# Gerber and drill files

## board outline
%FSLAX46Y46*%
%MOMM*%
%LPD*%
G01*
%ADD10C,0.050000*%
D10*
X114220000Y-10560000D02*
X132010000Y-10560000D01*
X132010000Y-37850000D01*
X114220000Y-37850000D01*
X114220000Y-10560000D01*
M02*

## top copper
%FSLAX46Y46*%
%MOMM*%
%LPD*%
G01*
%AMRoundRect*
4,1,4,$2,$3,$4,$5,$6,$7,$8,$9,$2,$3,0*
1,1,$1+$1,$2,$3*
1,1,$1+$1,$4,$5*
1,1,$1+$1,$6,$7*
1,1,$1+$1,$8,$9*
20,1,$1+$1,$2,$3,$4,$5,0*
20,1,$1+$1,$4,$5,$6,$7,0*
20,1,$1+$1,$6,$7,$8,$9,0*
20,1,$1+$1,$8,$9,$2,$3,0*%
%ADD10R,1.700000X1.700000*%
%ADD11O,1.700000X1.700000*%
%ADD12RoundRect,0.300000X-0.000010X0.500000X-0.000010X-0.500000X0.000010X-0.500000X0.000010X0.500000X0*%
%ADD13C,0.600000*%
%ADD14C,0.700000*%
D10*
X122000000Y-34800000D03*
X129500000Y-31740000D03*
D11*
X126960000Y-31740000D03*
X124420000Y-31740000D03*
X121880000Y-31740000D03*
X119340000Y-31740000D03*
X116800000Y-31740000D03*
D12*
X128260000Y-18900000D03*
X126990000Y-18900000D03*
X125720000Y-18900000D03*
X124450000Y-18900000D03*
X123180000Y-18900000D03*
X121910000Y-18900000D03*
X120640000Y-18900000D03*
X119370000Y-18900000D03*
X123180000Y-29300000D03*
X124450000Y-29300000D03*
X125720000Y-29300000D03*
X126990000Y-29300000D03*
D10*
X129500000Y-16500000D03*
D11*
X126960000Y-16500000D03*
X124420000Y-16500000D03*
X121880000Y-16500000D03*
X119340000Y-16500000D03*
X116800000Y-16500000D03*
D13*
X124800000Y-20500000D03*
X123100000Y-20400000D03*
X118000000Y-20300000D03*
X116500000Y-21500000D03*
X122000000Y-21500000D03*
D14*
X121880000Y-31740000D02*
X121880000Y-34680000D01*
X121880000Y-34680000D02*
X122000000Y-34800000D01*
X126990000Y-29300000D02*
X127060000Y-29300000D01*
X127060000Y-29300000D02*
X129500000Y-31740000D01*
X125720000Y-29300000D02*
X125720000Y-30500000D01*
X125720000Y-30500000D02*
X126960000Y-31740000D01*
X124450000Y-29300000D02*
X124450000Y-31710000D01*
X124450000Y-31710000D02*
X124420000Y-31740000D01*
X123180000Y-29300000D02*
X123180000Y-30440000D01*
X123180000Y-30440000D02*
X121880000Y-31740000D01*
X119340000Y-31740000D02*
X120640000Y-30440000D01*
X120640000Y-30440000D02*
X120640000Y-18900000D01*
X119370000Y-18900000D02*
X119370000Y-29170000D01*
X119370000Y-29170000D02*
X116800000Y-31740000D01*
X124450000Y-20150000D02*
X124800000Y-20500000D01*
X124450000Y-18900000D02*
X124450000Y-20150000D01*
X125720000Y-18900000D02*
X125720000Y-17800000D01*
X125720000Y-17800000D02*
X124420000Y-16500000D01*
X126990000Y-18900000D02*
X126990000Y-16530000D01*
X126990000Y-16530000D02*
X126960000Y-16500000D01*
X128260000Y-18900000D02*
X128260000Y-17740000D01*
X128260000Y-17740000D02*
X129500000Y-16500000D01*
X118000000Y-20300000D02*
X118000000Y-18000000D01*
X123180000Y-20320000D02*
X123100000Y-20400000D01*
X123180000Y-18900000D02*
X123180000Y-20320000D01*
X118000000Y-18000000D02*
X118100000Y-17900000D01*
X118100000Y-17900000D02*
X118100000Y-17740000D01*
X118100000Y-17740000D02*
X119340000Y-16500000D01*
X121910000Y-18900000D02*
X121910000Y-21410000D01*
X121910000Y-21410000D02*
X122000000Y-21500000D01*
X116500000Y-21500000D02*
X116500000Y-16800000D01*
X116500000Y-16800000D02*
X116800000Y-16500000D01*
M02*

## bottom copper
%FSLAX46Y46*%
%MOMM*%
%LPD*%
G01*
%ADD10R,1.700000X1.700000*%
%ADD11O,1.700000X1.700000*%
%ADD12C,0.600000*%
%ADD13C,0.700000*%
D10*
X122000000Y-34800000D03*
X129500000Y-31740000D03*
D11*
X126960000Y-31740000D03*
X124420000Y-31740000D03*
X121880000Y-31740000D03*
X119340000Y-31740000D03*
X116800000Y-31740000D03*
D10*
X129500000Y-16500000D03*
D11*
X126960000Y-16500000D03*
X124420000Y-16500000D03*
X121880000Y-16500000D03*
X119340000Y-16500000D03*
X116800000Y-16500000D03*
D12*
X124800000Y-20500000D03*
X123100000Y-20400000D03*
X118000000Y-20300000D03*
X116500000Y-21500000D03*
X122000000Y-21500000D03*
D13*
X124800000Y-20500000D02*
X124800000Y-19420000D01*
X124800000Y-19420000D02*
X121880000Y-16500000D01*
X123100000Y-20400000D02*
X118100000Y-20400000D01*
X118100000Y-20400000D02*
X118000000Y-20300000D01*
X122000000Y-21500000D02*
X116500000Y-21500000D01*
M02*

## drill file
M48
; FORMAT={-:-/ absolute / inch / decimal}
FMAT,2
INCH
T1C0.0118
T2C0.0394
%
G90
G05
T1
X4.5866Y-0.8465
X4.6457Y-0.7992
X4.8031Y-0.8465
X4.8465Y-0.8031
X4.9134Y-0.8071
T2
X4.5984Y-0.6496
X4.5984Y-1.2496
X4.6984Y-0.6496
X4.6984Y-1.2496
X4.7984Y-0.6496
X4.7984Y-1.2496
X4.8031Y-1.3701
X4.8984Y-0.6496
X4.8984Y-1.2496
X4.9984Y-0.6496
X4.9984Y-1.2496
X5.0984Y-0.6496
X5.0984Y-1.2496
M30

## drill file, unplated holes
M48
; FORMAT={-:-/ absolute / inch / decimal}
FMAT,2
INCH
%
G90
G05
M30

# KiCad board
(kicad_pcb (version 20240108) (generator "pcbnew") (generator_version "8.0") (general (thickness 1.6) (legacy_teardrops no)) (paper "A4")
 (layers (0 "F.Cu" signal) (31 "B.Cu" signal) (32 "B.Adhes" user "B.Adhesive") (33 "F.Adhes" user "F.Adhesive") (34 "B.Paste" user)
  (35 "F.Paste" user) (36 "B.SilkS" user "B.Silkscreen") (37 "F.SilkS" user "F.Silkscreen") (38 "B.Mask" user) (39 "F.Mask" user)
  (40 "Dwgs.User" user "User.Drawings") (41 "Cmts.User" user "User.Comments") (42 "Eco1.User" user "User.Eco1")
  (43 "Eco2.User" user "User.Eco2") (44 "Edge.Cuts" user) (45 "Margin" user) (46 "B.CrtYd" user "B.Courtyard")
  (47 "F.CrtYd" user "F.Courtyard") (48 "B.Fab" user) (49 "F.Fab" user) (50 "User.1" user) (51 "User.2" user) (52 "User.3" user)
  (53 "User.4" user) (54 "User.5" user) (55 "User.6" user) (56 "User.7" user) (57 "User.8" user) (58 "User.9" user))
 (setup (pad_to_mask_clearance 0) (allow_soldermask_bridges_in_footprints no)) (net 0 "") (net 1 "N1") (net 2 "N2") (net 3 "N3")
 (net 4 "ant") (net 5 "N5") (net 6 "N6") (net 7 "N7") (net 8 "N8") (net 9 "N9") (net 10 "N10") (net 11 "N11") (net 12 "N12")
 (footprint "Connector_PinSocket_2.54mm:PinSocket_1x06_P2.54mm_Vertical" (layer "F.Cu") (at 129.5 31.74 -90)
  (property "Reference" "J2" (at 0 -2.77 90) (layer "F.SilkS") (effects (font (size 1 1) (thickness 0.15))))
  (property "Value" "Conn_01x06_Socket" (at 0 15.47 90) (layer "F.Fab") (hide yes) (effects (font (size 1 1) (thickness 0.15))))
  (pad "1" thru_hole rect (at 0 0 270) (size 1.7 1.7) (drill 1) (layers "*.Cu" "*.Mask") (remove_unused_layers no) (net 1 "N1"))
  (pad "2" thru_hole oval (at 0 2.54 270) (size 1.7 1.7) (drill 1) (layers "*.Cu" "*.Mask") (remove_unused_layers no) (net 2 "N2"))
  (pad "3" thru_hole oval (at 0 5.08 270) (size 1.7 1.7) (drill 1) (layers "*.Cu" "*.Mask") (remove_unused_layers no) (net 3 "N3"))
  (pad "4" thru_hole oval (at 0 7.62 270) (size 1.7 1.7) (drill 1) (layers "*.Cu" "*.Mask") (remove_unused_layers no) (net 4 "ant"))
  (pad "5" thru_hole oval (at 0 10.16 270) (size 1.7 1.7) (drill 1) (layers "*.Cu" "*.Mask") (remove_unused_layers no) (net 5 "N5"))
  (pad "6" thru_hole oval (at 0 12.7 270) (size 1.7 1.7) (drill 1) (layers "*.Cu" "*.Mask") (remove_unused_layers no) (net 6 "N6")))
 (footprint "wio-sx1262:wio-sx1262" (layer "F.Cu") (at 129.59 18.6 180)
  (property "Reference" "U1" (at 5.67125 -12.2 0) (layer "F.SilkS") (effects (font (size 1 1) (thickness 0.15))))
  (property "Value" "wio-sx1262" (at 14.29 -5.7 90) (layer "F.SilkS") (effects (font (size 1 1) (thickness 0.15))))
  (pad "1" smd roundrect (at 1.33 -0.3 270) (size 1.6 0.6) (layers "F.Cu" "F.Paste" "F.Mask") (roundrect_rratio 0.5) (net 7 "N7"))
  (pad "2" smd roundrect (at 2.6 -0.3 270) (size 1.6 0.6) (layers "F.Cu" "F.Paste" "F.Mask") (roundrect_rratio 0.5) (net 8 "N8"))
  (pad "3" smd roundrect (at 3.87 -0.3 270) (size 1.6 0.6) (layers "F.Cu" "F.Paste" "F.Mask") (roundrect_rratio 0.5) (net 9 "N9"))
  (pad "4" smd roundrect (at 5.14 -0.3 270) (size 1.6 0.6) (layers "F.Cu" "F.Paste" "F.Mask") (roundrect_rratio 0.5) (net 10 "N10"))
  (pad "5" smd roundrect (at 6.41 -0.3 270) (size 1.6 0.6) (layers "F.Cu" "F.Paste" "F.Mask") (roundrect_rratio 0.5) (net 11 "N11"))
  (pad "6" smd roundrect (at 7.68 -0.3 270) (size 1.6 0.6) (layers "F.Cu" "F.Paste" "F.Mask") (roundrect_rratio 0.5) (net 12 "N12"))
  (pad "7" smd roundrect (at 8.95 -0.3 270) (size 1.6 0.6) (layers "F.Cu" "F.Paste" "F.Mask") (roundrect_rratio 0.5) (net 5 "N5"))
  (pad "8" smd roundrect (at 10.22 -0.3 270) (size 1.6 0.6) (layers "F.Cu" "F.Paste" "F.Mask") (roundrect_rratio 0.5) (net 6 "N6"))
  (pad "9" smd roundrect (at 6.41 -10.7 270) (size 1.6 0.6) (layers "F.Cu" "F.Paste" "F.Mask") (roundrect_rratio 0.5) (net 4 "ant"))
  (pad "10" smd roundrect (at 5.14 -10.7 270) (size 1.6 0.6) (layers "F.Cu" "F.Paste" "F.Mask") (roundrect_rratio 0.5) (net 3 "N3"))
  (pad "11" smd roundrect (at 3.87 -10.7 270) (size 1.6 0.6) (layers "F.Cu" "F.Paste" "F.Mask") (roundrect_rratio 0.5) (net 2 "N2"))
  (pad "12" smd roundrect (at 2.6 -10.7 270) (size 1.6 0.6) (layers "F.Cu" "F.Paste" "F.Mask") (roundrect_rratio 0.5) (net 1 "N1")))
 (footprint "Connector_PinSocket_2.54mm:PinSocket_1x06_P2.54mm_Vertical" (layer "F.Cu") (at 129.5 16.5 -90)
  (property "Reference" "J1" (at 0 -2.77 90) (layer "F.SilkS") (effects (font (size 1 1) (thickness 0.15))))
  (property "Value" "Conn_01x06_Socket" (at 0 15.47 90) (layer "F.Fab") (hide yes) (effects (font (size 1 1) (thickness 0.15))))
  (pad "1" thru_hole rect (at 0 0 270) (size 1.7 1.7) (drill 1) (layers "*.Cu" "*.Mask") (remove_unused_layers no) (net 7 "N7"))
  (pad "2" thru_hole oval (at 0 2.54 270) (size 1.7 1.7) (drill 1) (layers "*.Cu" "*.Mask") (remove_unused_layers no) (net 8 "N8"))
  (pad "3" thru_hole oval (at 0 5.08 270) (size 1.7 1.7) (drill 1) (layers "*.Cu" "*.Mask") (remove_unused_layers no) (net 9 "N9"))
  (pad "4" thru_hole oval (at 0 7.62 270) (size 1.7 1.7) (drill 1) (layers "*.Cu" "*.Mask") (remove_unused_layers no) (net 10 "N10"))
  (pad "5" thru_hole oval (at 0 10.16 270) (size 1.7 1.7) (drill 1) (layers "*.Cu" "*.Mask") (remove_unused_layers no) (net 11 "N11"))
  (pad "6" thru_hole oval (at 0 12.7 270) (size 1.7 1.7) (drill 1) (layers "*.Cu" "*.Mask") (remove_unused_layers no) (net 12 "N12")))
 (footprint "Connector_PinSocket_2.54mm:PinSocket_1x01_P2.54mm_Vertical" (layer "F.Cu") (at 122 34.8)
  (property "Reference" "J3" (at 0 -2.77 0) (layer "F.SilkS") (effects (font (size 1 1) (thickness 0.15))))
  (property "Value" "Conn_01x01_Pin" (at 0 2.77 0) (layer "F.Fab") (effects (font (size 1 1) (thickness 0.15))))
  (pad "1" thru_hole rect (at 0 0) (size 1.7 1.7) (drill 1) (layers "*.Cu" "*.Mask") (remove_unused_layers no) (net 4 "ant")))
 (gr_rect (start 114.22 10.56) (end 132.01 37.85) (stroke (width 0.05) (type default)) (fill none) (layer "Edge.Cuts"))
 (segment (start 124.45 18.9) (end 124.45 20.15) (width 0.7) (layer "F.Cu") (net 10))
 (segment (start 124.45 20.15) (end 124.8 20.5) (width 0.7) (layer "F.Cu") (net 10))
 (via (at 124.8 20.5) (size 0.6) (drill 0.3) (layers "F.Cu" "B.Cu") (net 10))
 (segment (start 124.8 19.42) (end 121.88 16.5) (width 0.7) (layer "B.Cu") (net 10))
 (segment (start 124.8 20.5) (end 124.8 19.42) (width 0.7) (layer "B.Cu") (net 10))
 (segment (start 126.99 18.9) (end 126.99 16.53) (width 0.7) (layer "F.Cu") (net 8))
 (segment (start 126.99 16.53) (end 126.96 16.5) (width 0.7) (layer "F.Cu") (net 8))
 (segment (start 121.91 18.9) (end 121.91 21.41) (width 0.7) (layer "F.Cu") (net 12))
 (segment (start 116.5 21.5) (end 116.5 16.8) (width 0.7) (layer "F.Cu") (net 12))
 (segment (start 116.5 16.8) (end 116.8 16.5) (width 0.7) (layer "F.Cu") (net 12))
 (segment (start 121.91 21.41) (end 122 21.5) (width 0.7) (layer "F.Cu") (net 12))
 (via (at 122 21.5) (size 0.6) (drill 0.3) (layers "F.Cu" "B.Cu") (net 12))
 (via (at 116.5 21.5) (size 0.6) (drill 0.3) (layers "F.Cu" "B.Cu") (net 12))
 (segment (start 122 21.5) (end 116.5 21.5) (width 0.7) (layer "B.Cu") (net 12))
 (segment (start 128.26 18.9) (end 128.26 17.74) (width 0.7) (layer "F.Cu") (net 7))
 (segment (start 128.26 17.74) (end 129.5 16.5) (width 0.7) (layer "F.Cu") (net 7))
 (segment (start 125.72 18.9) (end 125.72 17.8) (width 0.7) (layer "F.Cu") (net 9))
 (segment (start 125.72 17.8) (end 124.42 16.5) (width 0.7) (layer "F.Cu") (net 9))
 (segment (start 118 20.3) (end 118 18) (width 0.7) (layer "F.Cu") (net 11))
 (segment (start 118 18) (end 118.1 17.9) (width 0.7) (layer "F.Cu") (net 11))
 (segment (start 123.18 18.9) (end 123.18 20.32) (width 0.7) (layer "F.Cu") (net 11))
 (segment (start 118.1 17.9) (end 118.1 17.74) (width 0.7) (layer "F.Cu") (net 11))
 (segment (start 123.18 20.32) (end 123.1 20.4) (width 0.7) (layer "F.Cu") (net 11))
 (segment (start 118.1 17.74) (end 119.34 16.5) (width 0.7) (layer "F.Cu") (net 11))
 (via (at 123.1 20.4) (size 0.6) (drill 0.3) (layers "F.Cu" "B.Cu") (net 11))
 (via (at 118 20.3) (size 0.6) (drill 0.3) (layers "F.Cu" "B.Cu") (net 11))
 (segment (start 118.1 20.4) (end 118 20.3) (width 0.7) (layer "B.Cu") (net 11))
 (segment (start 123.1 20.4) (end 118.1 20.4) (width 0.7) (layer "B.Cu") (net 11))
 (segment (start 119.37 18.9) (end 119.37 29.17) (width 0.7) (layer "F.Cu") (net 6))
 (segment (start 119.37 29.17) (end 116.8 31.74) (width 0.7) (layer "F.Cu") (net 6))
 (segment (start 124.45 29.3) (end 124.45 31.71) (width 0.7) (layer "F.Cu") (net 3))
 (segment (start 124.45 31.71) (end 124.42 31.74) (width 0.7) (layer "F.Cu") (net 3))
 (segment (start 119.34 31.74) (end 120.64 30.44) (width 0.7) (layer "F.Cu") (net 5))
 (segment (start 120.64 30.44) (end 120.64 18.9) (width 0.7) (layer "F.Cu") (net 5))
 (segment (start 121.88 34.68) (end 122 34.8) (width 0.7) (layer "F.Cu") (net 4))
 (segment (start 123.18 29.3) (end 123.18 30.44) (width 0.7) (layer "F.Cu") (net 4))
 (segment (start 121.88 31.74) (end 121.88 34.68) (width 0.7) (layer "F.Cu") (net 4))
 (segment (start 123.18 30.44) (end 121.88 31.74) (width 0.7) (layer "F.Cu") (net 4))
 (segment (start 125.72 29.3) (end 125.72 30.5) (width 0.7) (layer "F.Cu") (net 2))
 (segment (start 125.72 30.5) (end 126.96 31.74) (width 0.7) (layer "F.Cu") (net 2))
 (segment (start 127.06 29.3) (end 129.5 31.74) (width 0.7) (layer "F.Cu") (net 1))
 (segment (start 126.99 29.3) (end 127.06 29.3) (width 0.7) (layer "F.Cu") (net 1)))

